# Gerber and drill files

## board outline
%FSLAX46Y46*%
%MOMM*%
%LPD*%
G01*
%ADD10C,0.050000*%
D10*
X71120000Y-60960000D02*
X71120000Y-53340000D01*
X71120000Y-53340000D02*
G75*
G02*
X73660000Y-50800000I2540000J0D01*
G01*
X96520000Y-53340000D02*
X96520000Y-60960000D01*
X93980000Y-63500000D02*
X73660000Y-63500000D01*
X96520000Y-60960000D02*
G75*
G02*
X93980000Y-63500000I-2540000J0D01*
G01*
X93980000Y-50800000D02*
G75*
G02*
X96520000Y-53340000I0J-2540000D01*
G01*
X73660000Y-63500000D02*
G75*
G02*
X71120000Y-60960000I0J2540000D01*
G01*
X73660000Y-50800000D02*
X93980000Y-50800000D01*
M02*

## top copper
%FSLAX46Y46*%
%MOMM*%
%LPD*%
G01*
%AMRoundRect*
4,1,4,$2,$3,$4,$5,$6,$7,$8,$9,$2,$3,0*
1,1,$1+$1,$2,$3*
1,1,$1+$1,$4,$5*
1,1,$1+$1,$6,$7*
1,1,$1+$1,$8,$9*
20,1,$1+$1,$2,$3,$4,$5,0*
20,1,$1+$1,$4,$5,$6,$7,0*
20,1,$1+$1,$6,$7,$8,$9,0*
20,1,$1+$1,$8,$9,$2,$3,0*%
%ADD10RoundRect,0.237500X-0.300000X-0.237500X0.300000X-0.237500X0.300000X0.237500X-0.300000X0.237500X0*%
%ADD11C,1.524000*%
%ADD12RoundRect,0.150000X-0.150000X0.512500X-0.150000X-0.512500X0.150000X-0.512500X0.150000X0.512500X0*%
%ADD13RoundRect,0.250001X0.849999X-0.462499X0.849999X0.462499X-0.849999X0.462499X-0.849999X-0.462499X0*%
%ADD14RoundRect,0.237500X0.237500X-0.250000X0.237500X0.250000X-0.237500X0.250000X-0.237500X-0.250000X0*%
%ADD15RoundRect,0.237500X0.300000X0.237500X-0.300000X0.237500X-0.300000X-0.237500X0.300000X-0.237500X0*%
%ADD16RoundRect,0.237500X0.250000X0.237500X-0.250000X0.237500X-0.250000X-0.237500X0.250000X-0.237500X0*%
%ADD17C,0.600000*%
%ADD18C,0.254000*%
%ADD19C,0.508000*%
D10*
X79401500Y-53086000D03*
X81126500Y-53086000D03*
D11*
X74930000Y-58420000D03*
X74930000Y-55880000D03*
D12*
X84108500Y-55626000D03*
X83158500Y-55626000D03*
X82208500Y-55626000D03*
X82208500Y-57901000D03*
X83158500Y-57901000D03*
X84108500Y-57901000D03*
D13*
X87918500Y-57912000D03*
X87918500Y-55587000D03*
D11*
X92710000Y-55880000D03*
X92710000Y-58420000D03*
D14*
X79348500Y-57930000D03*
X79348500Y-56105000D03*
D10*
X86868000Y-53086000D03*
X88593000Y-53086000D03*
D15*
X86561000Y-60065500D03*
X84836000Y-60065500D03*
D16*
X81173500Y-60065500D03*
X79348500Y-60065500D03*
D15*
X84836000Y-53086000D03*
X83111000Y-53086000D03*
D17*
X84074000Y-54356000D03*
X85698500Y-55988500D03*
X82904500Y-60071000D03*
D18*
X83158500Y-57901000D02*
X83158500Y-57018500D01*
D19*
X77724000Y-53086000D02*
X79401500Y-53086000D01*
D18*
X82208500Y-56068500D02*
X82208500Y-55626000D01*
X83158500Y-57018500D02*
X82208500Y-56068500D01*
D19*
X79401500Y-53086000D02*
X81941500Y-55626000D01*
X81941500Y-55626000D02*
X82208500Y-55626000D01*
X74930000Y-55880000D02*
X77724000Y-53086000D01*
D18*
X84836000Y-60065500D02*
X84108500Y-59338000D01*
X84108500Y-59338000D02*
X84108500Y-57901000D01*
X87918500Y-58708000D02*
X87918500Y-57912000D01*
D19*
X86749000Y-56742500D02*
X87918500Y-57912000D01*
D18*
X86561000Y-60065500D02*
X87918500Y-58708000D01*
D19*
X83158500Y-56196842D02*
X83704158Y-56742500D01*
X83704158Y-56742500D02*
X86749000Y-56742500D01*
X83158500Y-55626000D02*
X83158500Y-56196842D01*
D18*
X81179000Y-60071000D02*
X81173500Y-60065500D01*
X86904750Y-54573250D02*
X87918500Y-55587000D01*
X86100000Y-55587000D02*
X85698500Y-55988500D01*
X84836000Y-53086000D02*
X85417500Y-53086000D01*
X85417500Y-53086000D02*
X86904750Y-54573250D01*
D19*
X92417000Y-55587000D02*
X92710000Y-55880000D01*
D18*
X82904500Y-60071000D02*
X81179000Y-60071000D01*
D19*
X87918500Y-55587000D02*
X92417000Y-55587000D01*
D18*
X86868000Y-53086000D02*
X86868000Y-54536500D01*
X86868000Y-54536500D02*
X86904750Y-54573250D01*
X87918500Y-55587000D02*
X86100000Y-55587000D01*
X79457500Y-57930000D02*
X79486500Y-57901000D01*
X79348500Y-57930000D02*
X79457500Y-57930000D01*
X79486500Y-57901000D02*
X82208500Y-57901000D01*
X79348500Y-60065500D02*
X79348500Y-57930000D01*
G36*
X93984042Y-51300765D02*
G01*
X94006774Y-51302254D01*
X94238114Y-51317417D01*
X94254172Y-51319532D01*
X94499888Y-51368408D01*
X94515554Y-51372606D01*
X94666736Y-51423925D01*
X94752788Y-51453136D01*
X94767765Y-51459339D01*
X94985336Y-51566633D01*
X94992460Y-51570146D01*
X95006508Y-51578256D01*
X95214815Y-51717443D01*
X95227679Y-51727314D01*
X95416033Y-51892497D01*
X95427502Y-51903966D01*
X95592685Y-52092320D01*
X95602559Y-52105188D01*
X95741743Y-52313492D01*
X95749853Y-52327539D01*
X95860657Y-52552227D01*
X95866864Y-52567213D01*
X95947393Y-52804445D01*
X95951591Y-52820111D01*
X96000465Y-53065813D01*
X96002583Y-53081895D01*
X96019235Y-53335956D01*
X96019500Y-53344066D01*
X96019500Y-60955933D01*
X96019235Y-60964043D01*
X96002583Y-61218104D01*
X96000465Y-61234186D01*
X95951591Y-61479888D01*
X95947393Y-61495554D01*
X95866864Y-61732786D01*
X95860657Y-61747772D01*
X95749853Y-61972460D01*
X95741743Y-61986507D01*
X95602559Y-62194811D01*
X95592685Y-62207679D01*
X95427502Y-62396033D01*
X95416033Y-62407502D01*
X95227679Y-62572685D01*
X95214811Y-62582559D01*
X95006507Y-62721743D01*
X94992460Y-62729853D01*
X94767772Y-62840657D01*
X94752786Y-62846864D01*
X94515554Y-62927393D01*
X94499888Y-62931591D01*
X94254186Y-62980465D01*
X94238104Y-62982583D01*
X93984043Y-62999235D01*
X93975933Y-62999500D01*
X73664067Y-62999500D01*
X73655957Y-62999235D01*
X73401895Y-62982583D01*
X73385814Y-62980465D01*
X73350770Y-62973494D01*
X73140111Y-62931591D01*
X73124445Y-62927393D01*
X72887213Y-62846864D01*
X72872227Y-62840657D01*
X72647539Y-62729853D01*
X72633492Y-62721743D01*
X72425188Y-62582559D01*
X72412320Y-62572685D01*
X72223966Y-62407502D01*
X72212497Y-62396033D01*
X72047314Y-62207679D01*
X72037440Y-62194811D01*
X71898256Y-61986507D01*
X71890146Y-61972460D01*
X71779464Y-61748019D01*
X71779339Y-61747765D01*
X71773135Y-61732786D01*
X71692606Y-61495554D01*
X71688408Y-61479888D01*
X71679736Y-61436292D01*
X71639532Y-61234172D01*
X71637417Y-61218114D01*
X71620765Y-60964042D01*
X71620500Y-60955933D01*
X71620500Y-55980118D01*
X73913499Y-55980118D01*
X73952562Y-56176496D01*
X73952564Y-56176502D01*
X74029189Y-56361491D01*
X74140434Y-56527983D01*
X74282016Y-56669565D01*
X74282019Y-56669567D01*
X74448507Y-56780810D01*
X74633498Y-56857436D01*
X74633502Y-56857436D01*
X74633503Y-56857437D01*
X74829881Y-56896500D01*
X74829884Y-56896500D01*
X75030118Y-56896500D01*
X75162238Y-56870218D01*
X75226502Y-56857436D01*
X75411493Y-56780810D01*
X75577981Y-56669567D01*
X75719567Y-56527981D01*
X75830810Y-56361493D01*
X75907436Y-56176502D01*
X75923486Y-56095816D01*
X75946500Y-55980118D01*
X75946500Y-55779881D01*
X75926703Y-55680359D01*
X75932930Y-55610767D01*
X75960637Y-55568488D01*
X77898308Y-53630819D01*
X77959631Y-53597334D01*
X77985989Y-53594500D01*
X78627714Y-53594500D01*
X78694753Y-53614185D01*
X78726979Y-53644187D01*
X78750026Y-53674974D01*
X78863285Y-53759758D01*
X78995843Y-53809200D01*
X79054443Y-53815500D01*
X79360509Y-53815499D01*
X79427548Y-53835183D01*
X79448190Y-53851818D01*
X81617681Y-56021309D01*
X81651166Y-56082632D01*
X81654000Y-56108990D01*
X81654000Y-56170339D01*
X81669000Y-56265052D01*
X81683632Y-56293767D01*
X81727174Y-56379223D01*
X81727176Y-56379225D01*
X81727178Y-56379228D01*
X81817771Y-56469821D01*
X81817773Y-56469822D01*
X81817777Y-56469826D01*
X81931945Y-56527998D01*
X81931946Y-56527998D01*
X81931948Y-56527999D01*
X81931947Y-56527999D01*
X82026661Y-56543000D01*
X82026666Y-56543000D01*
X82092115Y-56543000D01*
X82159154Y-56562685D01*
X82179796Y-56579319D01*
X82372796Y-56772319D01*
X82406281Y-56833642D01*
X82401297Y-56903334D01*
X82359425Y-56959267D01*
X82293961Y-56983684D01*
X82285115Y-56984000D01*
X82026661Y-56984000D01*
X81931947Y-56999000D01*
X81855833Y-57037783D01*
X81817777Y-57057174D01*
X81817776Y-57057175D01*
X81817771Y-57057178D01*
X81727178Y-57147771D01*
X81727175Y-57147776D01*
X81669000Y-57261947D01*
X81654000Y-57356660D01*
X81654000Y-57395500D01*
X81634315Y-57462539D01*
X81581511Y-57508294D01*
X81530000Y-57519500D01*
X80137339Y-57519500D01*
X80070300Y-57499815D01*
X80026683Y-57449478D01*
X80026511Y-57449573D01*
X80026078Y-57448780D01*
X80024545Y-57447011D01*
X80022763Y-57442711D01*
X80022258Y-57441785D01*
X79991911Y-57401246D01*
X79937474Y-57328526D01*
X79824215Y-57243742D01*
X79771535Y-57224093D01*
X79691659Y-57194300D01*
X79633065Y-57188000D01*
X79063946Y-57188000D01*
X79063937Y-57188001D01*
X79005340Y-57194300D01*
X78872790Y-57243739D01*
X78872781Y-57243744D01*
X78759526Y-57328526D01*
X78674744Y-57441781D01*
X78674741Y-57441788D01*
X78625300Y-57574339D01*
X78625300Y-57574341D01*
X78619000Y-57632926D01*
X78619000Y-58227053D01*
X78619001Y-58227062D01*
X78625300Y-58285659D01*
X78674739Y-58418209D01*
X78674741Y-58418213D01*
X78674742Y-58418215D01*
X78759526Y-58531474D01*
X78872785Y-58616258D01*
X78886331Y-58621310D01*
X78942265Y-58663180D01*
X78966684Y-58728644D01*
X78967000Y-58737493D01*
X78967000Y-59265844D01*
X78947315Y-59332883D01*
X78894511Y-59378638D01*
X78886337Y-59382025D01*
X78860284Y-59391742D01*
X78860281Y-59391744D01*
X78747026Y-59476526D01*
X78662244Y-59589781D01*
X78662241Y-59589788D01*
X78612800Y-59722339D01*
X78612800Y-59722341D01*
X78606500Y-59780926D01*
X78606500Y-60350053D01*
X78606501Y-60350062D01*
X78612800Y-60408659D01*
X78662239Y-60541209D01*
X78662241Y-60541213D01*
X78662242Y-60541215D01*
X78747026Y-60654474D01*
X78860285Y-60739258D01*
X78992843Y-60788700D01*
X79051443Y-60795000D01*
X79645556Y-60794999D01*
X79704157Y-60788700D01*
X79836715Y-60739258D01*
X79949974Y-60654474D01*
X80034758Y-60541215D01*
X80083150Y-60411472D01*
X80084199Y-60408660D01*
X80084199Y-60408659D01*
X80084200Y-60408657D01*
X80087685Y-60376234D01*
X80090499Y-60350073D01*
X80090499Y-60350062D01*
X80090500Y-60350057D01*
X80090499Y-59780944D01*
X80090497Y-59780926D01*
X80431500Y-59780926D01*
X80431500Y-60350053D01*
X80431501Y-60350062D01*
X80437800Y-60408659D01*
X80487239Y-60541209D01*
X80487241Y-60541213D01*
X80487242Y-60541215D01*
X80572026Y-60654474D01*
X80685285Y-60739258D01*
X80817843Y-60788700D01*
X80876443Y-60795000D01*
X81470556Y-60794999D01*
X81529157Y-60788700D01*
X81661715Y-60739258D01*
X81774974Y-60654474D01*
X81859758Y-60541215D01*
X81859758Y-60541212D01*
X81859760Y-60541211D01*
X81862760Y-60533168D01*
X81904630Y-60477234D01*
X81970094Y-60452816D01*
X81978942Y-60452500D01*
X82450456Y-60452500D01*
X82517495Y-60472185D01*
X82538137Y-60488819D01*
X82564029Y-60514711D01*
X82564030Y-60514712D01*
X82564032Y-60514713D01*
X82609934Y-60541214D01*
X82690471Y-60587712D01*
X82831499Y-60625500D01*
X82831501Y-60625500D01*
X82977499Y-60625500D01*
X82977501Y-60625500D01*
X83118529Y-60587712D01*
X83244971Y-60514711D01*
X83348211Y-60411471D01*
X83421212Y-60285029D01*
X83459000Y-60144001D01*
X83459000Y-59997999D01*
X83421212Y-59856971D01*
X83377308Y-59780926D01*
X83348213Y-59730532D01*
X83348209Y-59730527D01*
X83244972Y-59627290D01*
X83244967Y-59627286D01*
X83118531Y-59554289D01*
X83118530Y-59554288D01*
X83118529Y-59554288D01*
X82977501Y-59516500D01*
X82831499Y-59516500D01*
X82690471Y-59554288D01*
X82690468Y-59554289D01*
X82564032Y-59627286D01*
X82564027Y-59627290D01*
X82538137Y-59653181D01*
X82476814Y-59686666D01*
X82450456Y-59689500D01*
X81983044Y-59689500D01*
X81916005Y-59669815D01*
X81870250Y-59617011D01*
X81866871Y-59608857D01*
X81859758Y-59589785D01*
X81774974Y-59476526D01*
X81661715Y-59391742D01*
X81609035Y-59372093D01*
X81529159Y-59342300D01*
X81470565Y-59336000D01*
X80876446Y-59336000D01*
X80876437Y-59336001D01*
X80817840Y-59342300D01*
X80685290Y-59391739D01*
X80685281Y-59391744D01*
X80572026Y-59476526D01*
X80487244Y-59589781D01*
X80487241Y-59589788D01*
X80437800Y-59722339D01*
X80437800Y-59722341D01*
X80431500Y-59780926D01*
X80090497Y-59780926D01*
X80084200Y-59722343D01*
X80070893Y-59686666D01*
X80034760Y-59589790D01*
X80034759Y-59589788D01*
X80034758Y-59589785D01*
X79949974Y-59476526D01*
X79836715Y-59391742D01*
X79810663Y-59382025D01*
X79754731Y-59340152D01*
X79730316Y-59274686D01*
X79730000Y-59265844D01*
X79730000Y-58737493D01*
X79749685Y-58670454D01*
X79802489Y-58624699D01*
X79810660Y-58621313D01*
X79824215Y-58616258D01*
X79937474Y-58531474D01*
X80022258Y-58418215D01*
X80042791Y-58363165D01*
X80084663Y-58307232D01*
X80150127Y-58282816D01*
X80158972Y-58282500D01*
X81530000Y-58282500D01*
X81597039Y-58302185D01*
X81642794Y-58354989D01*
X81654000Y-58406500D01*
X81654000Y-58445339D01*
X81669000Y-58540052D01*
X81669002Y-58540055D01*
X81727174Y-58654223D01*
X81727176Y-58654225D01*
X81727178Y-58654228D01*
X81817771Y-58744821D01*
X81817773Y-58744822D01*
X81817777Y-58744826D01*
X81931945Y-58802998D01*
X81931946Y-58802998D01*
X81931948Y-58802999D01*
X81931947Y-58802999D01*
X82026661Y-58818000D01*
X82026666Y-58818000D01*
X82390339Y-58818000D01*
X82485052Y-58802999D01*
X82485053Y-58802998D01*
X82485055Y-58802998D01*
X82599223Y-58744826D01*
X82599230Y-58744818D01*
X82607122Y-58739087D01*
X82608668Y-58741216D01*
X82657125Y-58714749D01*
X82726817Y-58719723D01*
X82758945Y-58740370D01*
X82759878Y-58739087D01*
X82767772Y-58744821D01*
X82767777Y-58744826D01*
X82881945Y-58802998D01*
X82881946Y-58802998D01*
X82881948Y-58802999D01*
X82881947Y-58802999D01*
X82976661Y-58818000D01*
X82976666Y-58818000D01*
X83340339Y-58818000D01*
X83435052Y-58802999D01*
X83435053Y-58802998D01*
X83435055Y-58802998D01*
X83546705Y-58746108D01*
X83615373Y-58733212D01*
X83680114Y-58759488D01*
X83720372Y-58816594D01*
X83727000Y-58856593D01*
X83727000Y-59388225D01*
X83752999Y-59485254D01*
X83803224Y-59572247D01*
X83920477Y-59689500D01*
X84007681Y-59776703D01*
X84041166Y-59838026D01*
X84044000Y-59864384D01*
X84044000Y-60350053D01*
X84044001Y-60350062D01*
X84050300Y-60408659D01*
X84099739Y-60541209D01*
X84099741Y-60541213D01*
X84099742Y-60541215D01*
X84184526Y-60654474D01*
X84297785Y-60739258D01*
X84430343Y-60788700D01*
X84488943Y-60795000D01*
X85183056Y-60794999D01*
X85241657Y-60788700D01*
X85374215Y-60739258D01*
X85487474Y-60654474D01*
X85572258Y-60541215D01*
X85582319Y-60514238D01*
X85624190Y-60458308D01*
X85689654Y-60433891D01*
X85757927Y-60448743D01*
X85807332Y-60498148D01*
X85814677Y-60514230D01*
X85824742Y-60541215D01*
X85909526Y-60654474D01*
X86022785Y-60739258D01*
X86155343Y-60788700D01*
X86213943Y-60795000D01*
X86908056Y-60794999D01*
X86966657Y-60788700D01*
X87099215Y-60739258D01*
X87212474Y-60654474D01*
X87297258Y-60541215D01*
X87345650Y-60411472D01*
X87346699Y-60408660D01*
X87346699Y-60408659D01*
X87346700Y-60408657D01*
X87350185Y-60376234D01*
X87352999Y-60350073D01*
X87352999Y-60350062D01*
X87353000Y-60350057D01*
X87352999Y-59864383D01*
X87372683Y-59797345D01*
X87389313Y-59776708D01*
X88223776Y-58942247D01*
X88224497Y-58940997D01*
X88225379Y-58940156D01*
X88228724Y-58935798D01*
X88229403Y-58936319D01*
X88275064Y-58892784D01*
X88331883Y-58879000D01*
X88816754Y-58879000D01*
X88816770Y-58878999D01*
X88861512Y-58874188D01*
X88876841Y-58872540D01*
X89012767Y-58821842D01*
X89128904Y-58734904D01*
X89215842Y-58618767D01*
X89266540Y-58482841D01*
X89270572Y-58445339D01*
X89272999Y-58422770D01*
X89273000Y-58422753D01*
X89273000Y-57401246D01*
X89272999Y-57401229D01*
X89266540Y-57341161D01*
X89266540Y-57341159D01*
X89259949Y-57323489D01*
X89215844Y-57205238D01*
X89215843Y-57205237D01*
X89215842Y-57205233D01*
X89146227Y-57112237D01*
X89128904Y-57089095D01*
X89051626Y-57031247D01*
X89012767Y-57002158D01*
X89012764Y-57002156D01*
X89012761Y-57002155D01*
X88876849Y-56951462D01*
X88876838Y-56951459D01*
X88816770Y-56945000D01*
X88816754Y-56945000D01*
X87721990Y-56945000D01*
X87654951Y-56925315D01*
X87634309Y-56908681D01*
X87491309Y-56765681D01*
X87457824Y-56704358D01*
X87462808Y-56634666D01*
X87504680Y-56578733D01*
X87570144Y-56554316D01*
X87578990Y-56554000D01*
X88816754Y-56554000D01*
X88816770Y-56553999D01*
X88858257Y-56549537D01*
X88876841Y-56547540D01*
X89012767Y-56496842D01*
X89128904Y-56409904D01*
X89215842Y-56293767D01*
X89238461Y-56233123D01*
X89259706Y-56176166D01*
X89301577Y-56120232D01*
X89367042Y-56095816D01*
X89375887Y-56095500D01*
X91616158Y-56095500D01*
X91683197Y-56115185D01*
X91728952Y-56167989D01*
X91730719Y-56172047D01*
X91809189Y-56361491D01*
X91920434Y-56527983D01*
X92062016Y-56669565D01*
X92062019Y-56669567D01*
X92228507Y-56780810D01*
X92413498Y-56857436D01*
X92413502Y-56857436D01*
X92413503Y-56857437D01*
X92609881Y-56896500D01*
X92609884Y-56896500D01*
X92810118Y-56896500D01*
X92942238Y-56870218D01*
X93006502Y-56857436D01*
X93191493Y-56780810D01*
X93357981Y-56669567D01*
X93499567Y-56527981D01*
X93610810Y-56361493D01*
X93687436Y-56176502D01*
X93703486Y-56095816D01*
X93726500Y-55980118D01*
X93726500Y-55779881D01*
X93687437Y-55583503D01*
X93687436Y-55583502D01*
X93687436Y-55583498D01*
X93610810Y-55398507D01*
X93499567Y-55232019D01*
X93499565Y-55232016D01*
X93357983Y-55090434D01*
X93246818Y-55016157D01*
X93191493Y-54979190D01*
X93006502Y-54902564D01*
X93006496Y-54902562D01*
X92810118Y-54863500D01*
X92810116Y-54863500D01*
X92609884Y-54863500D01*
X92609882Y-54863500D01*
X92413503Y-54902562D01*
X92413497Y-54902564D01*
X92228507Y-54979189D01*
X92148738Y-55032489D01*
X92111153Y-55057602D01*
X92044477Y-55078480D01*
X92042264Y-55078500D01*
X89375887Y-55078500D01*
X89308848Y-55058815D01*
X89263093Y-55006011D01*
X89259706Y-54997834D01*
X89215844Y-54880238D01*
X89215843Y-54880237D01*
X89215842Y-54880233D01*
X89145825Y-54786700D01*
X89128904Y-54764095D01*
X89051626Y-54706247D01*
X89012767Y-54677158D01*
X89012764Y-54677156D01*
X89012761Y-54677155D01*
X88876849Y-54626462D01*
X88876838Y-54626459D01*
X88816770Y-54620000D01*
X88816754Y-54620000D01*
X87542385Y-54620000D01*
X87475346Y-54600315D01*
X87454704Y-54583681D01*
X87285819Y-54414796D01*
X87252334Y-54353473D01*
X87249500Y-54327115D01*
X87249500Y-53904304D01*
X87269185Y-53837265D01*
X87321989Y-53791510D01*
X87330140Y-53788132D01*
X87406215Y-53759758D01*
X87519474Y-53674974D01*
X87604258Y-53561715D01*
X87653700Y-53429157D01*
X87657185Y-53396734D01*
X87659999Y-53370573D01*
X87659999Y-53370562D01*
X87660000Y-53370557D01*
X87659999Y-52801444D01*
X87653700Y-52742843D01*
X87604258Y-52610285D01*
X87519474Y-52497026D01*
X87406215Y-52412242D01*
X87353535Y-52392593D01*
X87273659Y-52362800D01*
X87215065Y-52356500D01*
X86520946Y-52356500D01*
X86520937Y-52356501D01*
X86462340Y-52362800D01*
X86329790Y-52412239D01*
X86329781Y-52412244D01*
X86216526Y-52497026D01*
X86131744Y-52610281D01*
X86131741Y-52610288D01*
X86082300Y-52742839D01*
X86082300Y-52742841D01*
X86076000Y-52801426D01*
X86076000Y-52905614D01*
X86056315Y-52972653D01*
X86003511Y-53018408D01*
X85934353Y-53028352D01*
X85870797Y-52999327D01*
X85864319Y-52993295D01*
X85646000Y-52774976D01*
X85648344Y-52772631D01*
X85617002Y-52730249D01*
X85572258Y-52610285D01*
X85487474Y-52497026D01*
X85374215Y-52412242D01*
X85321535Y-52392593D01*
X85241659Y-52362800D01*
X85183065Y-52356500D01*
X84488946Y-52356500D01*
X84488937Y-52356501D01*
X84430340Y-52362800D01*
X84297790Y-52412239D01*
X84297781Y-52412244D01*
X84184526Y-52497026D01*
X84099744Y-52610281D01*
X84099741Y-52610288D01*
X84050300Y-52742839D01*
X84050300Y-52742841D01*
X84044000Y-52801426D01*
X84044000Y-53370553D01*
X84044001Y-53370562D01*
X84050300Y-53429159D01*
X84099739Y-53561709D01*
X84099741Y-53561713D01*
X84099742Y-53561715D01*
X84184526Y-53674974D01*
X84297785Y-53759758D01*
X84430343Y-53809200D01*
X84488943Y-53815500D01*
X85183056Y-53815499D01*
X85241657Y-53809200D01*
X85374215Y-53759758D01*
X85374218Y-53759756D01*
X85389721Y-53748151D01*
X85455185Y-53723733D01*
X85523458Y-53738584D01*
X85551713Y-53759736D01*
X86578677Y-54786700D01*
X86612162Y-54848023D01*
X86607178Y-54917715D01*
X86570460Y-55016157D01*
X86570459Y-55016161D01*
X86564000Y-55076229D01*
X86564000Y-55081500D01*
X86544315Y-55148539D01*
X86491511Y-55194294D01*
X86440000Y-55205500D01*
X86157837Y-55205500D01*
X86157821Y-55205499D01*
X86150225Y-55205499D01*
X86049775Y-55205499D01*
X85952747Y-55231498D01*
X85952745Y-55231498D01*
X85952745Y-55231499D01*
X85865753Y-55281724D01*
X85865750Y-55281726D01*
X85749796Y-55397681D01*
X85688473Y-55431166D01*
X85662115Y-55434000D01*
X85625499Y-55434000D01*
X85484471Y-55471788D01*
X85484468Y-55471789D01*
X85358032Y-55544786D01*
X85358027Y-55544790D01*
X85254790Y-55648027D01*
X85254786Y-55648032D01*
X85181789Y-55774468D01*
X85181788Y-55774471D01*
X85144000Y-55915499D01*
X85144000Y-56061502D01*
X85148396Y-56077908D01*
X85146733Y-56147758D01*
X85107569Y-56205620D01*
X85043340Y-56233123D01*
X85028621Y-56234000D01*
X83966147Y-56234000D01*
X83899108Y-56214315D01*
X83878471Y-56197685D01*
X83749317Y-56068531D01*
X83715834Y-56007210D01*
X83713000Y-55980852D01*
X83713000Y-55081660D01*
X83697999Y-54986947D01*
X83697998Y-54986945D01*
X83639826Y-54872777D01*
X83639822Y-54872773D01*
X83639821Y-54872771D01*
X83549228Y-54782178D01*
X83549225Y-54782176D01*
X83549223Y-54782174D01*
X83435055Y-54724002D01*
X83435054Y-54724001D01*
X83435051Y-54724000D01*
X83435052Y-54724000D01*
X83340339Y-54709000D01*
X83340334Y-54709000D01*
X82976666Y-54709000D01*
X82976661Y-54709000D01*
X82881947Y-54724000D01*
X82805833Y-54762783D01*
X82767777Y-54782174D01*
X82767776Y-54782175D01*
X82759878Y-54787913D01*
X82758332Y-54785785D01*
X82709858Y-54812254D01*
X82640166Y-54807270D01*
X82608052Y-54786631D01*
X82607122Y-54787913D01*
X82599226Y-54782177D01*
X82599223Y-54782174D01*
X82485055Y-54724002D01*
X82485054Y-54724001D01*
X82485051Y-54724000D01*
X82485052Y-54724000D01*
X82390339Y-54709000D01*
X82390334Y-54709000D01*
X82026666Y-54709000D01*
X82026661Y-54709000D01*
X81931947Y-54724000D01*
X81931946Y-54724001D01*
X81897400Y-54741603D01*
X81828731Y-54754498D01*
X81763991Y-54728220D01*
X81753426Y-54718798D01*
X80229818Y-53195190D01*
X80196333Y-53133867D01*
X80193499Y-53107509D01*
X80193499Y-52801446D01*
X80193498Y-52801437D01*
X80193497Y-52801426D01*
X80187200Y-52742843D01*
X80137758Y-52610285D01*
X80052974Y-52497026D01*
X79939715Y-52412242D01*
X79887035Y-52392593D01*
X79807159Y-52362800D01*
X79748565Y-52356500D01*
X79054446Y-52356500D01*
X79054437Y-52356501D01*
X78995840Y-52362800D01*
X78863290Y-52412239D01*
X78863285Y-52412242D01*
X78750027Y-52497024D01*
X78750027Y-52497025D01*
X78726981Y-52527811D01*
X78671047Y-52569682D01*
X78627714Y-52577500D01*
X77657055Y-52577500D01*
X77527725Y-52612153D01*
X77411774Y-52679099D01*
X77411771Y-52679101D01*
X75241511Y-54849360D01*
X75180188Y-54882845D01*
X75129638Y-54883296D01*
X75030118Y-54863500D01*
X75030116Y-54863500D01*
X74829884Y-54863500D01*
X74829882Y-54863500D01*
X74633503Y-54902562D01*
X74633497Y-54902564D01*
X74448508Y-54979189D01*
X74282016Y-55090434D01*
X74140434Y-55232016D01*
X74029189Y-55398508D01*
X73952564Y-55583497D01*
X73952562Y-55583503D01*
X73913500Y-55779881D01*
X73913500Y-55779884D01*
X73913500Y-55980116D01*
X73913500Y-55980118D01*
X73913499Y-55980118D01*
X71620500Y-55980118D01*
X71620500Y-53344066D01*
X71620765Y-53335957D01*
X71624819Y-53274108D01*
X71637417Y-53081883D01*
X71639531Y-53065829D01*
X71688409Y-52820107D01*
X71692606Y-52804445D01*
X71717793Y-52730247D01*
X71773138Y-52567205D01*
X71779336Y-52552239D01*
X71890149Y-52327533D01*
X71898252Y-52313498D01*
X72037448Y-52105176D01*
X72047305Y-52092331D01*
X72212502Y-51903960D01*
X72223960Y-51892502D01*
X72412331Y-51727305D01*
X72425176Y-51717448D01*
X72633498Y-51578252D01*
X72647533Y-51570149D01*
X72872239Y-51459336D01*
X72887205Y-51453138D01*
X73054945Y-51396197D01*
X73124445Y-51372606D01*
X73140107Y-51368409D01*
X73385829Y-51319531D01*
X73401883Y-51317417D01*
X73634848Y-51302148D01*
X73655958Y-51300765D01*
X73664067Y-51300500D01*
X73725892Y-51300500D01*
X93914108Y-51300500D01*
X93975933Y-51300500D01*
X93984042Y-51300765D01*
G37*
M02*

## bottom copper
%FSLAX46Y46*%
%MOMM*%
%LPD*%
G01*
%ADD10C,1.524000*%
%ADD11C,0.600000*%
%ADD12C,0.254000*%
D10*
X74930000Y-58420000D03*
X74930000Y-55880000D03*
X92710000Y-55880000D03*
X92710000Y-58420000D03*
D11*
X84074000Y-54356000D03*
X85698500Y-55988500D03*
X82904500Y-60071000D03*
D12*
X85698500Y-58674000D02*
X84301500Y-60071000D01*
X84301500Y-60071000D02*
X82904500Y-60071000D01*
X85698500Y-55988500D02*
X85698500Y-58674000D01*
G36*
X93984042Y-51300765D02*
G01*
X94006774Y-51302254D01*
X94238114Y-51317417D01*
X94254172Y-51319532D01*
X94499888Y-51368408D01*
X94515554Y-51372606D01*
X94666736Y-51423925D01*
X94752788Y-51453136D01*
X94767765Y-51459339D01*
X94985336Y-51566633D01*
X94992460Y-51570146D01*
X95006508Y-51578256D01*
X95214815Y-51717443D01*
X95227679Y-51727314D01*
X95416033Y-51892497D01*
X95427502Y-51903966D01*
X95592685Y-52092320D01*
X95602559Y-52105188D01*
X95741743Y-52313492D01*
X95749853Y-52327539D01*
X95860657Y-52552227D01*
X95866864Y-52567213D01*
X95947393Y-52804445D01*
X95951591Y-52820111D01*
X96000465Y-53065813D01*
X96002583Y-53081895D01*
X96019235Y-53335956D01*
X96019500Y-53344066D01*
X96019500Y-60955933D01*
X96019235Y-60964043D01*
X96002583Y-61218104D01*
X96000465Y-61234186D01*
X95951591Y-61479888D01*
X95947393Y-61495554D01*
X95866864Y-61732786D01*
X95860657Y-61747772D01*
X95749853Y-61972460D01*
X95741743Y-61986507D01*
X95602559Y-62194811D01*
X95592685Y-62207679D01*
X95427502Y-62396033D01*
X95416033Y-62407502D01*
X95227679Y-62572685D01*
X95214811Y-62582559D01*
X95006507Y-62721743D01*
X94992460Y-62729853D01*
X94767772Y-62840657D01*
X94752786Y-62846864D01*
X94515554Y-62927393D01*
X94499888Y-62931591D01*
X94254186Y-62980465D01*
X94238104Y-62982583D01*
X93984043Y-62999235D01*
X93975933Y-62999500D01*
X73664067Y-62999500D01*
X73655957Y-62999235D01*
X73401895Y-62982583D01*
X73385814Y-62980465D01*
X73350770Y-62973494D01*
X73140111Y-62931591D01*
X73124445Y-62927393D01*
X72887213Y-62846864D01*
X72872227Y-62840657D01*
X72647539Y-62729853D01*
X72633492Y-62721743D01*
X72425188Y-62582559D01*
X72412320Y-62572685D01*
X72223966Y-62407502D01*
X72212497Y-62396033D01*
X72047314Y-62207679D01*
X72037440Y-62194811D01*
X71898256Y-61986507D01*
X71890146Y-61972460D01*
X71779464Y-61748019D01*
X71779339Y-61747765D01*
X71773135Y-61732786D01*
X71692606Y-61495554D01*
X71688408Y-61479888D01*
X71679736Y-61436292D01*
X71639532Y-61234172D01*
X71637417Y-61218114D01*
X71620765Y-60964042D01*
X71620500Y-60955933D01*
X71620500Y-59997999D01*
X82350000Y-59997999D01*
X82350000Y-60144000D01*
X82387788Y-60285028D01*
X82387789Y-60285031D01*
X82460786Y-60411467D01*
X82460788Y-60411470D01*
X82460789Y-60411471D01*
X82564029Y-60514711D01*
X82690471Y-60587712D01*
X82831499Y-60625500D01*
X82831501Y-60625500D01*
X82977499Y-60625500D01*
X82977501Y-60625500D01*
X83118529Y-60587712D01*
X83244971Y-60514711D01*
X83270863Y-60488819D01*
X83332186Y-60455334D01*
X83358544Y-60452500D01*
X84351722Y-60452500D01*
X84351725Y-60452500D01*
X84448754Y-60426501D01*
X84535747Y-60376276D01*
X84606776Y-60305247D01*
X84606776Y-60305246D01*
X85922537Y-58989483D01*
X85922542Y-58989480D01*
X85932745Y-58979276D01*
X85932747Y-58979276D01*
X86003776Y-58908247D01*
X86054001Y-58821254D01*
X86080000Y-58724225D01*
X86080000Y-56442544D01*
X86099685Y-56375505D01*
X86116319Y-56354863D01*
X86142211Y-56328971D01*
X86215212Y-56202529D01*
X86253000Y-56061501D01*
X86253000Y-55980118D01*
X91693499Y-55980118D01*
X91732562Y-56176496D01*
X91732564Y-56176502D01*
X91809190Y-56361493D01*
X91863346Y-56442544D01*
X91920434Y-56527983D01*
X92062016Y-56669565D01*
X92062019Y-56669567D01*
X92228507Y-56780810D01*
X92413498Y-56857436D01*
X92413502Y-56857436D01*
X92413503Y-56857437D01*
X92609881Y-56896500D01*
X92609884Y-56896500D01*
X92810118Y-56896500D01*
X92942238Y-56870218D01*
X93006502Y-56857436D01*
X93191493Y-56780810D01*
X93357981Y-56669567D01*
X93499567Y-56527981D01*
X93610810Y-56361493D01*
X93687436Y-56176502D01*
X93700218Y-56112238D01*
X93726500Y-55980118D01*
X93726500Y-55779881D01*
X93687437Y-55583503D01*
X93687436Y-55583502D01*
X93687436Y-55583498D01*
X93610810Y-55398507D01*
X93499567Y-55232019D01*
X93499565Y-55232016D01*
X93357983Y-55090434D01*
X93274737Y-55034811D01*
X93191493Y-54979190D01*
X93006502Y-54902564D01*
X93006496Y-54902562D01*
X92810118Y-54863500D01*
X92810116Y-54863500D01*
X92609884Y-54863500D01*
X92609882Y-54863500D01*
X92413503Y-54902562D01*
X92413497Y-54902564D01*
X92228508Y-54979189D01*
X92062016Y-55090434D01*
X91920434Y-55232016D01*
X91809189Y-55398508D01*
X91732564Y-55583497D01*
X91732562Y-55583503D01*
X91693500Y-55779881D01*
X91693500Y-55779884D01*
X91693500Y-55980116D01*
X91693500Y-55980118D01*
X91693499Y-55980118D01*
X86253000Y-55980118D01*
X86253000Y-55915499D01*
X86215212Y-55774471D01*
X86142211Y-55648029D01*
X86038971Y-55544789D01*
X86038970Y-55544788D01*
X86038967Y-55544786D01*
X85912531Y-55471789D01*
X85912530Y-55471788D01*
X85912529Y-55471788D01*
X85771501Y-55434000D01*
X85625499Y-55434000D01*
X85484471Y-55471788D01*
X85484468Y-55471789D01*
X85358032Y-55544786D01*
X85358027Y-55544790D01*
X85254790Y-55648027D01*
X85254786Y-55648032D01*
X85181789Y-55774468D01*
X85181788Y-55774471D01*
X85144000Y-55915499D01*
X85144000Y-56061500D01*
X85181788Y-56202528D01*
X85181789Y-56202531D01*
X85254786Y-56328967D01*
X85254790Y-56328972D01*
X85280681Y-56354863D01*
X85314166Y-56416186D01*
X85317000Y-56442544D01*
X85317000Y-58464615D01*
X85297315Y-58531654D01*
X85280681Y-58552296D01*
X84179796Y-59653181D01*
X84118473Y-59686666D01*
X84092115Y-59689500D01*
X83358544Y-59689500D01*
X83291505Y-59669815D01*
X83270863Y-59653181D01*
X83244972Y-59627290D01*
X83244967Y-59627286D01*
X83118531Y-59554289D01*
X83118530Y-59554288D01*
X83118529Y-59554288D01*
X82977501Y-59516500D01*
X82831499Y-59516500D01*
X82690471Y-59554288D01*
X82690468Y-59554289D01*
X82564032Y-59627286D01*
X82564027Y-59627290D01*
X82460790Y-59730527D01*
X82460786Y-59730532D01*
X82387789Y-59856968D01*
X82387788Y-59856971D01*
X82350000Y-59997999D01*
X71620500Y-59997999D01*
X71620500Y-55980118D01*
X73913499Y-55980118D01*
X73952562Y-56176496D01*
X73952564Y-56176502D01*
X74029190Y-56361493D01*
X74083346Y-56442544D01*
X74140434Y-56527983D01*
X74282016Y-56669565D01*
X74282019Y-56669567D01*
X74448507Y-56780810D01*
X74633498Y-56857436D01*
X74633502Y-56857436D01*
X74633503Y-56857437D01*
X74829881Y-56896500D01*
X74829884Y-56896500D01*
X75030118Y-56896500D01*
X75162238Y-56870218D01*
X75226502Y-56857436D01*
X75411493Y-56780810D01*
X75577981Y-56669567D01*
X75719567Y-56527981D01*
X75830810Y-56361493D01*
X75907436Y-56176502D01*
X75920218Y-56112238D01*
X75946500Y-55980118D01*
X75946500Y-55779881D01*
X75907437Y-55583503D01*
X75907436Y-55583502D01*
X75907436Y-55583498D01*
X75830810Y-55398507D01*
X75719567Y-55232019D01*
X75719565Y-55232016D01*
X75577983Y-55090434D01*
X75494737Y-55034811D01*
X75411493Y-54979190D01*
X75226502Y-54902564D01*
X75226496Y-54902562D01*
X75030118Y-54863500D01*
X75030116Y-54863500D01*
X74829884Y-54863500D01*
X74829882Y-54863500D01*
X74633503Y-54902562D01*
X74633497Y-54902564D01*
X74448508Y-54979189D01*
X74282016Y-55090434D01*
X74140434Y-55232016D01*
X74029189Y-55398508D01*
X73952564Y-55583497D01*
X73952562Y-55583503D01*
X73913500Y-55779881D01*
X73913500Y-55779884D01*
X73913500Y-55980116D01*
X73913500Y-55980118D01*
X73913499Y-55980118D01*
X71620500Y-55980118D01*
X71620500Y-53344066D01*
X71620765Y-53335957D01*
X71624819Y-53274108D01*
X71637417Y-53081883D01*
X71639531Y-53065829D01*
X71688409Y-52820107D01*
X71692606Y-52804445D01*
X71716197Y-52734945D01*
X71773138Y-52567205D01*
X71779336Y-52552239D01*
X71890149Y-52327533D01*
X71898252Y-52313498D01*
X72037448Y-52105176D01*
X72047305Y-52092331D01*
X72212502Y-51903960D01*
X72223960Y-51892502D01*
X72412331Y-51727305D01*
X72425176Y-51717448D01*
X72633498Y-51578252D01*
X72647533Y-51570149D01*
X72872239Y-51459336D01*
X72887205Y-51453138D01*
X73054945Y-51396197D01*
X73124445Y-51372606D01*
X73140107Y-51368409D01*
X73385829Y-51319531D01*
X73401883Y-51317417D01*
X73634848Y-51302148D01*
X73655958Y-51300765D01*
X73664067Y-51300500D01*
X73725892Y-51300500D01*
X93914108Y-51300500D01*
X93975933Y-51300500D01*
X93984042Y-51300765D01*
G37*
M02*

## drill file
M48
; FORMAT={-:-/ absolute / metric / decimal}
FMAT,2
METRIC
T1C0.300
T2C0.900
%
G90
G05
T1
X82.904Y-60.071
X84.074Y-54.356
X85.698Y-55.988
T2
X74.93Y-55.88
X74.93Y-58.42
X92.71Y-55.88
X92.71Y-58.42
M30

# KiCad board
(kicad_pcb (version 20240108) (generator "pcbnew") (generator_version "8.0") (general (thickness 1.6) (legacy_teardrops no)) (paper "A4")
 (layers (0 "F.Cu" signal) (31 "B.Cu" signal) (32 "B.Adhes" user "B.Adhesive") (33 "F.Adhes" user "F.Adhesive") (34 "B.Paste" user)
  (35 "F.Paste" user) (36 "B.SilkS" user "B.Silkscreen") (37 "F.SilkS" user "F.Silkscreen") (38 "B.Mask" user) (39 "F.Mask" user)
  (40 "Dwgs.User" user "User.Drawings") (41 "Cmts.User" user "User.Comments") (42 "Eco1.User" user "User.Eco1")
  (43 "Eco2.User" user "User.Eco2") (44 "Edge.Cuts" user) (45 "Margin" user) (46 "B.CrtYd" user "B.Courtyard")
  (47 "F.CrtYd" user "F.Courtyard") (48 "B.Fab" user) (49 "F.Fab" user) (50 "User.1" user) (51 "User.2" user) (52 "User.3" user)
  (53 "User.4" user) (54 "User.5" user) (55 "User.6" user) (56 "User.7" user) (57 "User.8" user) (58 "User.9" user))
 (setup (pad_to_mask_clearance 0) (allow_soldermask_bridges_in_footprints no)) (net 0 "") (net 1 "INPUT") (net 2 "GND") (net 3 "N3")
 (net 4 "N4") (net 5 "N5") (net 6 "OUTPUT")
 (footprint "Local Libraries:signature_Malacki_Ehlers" (layer "F.Cu") (at 83.312 62.23)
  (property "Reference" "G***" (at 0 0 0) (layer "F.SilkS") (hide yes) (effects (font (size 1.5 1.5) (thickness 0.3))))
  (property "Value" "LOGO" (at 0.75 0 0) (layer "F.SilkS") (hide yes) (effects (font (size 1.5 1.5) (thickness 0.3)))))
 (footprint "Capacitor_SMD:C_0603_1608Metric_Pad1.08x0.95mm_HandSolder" (layer "F.Cu") (at 80.264 53.086)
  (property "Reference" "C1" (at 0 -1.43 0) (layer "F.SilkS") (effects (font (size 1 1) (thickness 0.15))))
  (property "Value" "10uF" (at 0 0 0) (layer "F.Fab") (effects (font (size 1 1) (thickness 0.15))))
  (pad "1" smd roundrect (at -0.8625 0) (size 1.075 0.95) (layers "F.Cu" "F.Paste" "F.Mask") (roundrect_rratio 0.25) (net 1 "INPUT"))
  (pad "2" smd roundrect (at 0.8625 0) (size 1.075 0.95) (layers "F.Cu" "F.Paste" "F.Mask") (roundrect_rratio 0.25) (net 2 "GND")))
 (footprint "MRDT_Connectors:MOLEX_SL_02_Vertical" (layer "F.Cu") (at 74.93 58.42 90)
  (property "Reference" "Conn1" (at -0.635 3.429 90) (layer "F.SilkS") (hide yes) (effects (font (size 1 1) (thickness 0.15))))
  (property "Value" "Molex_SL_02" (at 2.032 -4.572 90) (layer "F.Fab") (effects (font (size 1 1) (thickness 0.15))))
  (pad "1" thru_hole circle (at 0 0 90) (size 1.524 1.524) (drill 0.9) (layers "*.Cu" "*.Mask") (remove_unused_layers no) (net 2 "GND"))
  (pad "2" thru_hole circle (at 2.54 0 90) (size 1.524 1.524) (drill 0.9) (layers "*.Cu" "*.Mask") (remove_unused_layers no) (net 1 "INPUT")))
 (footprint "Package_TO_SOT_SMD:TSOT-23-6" (layer "F.Cu") (at 83.1585 56.7635 -90)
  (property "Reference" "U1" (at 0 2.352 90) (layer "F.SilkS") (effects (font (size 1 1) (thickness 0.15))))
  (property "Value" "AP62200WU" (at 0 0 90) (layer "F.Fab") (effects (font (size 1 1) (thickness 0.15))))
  (pad "1" smd roundrect (at -1.1375 -0.95 270) (size 1.325 0.6) (layers "F.Cu" "F.Paste" "F.Mask") (roundrect_rratio 0.25) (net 2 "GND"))
  (pad "2" smd roundrect (at -1.1375 0 270) (size 1.325 0.6) (layers "F.Cu" "F.Paste" "F.Mask") (roundrect_rratio 0.25) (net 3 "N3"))
  (pad "3" smd roundrect (at -1.1375 0.95 270) (size 1.325 0.6) (layers "F.Cu" "F.Paste" "F.Mask") (roundrect_rratio 0.25) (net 1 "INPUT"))
  (pad "4" smd roundrect (at 1.1375 0.95 270) (size 1.325 0.6) (layers "F.Cu" "F.Paste" "F.Mask") (roundrect_rratio 0.25) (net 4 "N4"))
  (pad "5" smd roundrect (at 1.1375 0 270) (size 1.325 0.6) (layers "F.Cu" "F.Paste" "F.Mask") (roundrect_rratio 0.25) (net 1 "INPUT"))
  (pad "6" smd roundrect (at 1.1375 -0.95 270) (size 1.325 0.6) (layers "F.Cu" "F.Paste" "F.Mask") (roundrect_rratio 0.25) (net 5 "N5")))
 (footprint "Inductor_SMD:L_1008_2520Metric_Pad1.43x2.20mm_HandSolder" (layer "F.Cu") (at 87.9185 56.7495 90)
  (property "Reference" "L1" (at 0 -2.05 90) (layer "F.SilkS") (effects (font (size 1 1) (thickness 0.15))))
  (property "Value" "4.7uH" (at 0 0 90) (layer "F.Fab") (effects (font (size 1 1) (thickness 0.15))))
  (pad "1" smd roundrect (at -1.1625 0 90) (size 1.425 2.2) (layers "F.Cu" "F.Paste" "F.Mask") (roundrect_rratio 0.175439) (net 3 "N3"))
  (pad "2" smd roundrect (at 1.1625 0 90) (size 1.425 2.2) (layers "F.Cu" "F.Paste" "F.Mask") (roundrect_rratio 0.175439) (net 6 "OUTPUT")))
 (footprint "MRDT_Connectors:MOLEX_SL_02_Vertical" (layer "F.Cu") (at 92.71 55.88 -90)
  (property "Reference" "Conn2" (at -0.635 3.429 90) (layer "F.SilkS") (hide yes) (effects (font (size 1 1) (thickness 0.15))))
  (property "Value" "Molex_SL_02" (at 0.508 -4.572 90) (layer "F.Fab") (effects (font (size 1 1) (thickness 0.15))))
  (pad "1" thru_hole circle (at 0 0 270) (size 1.524 1.524) (drill 0.9) (layers "*.Cu" "*.Mask") (remove_unused_layers no) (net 6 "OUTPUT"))
  (pad "2" thru_hole circle (at 2.54 0 270) (size 1.524 1.524) (drill 0.9) (layers "*.Cu" "*.Mask") (remove_unused_layers no) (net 2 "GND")))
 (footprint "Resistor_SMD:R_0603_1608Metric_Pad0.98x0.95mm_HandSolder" (layer "F.Cu") (at 79.3485 57.0175 90)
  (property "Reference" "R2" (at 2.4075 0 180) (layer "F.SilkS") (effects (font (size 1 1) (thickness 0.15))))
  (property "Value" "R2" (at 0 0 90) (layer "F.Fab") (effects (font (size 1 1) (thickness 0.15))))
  (pad "1" smd roundrect (at -0.9125 0 90) (size 0.975 0.95) (layers "F.Cu" "F.Paste" "F.Mask") (roundrect_rratio 0.25) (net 4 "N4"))
  (pad "2" smd roundrect (at 0.9125 0 90) (size 0.975 0.95) (layers "F.Cu" "F.Paste" "F.Mask") (roundrect_rratio 0.25) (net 2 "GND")))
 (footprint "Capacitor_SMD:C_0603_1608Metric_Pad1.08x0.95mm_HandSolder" (layer "F.Cu") (at 87.7305 53.086)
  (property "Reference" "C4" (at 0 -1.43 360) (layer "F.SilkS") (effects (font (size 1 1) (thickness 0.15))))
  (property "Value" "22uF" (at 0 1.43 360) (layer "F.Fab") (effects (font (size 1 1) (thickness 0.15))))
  (pad "1" smd roundrect (at -0.8625 0) (size 1.075 0.95) (layers "F.Cu" "F.Paste" "F.Mask") (roundrect_rratio 0.25) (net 6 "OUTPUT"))
  (pad "2" smd roundrect (at 0.8625 0) (size 1.075 0.95) (layers "F.Cu" "F.Paste" "F.Mask") (roundrect_rratio 0.25) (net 2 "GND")))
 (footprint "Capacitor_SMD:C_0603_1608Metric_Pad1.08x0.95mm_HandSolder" (layer "F.Cu") (at 85.6985 60.0655 180)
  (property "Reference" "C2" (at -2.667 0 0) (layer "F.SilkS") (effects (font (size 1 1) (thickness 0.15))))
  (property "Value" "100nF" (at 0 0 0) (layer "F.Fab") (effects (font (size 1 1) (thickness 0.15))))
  (pad "1" smd roundrect (at -0.8625 0 180) (size 1.075 0.95) (layers "F.Cu" "F.Paste" "F.Mask") (roundrect_rratio 0.25) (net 3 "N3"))
  (pad "2" smd roundrect (at 0.8625 0 180) (size 1.075 0.95) (layers "F.Cu" "F.Paste" "F.Mask") (roundrect_rratio 0.25) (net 5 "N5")))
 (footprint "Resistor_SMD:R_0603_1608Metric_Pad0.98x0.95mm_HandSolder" (layer "F.Cu") (at 80.261 60.0655 180)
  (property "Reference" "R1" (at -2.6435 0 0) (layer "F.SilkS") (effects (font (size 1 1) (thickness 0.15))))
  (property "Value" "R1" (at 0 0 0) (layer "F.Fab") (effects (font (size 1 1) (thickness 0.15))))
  (pad "1" smd roundrect (at -0.9125 0 180) (size 0.975 0.95) (layers "F.Cu" "F.Paste" "F.Mask") (roundrect_rratio 0.25) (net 6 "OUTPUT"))
  (pad "2" smd roundrect (at 0.9125 0 180) (size 0.975 0.95) (layers "F.Cu" "F.Paste" "F.Mask") (roundrect_rratio 0.25) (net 4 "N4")))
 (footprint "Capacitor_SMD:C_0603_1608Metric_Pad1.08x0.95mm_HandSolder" (layer "F.Cu") (at 83.9735 53.086 180)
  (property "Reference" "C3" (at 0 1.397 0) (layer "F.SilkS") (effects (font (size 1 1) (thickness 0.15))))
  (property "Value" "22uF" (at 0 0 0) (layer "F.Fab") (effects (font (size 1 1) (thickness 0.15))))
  (pad "1" smd roundrect (at -0.8625 0 180) (size 1.075 0.95) (layers "F.Cu" "F.Paste" "F.Mask") (roundrect_rratio 0.25) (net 6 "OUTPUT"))
  (pad "2" smd roundrect (at 0.8625 0 180) (size 1.075 0.95) (layers "F.Cu" "F.Paste" "F.Mask") (roundrect_rratio 0.25) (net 2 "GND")))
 (gr_line (start 71.12 60.96) (end 71.12 53.34) (stroke (width 0.05) (type default)) (layer "Edge.Cuts"))
 (gr_arc (start 71.12 53.34) (mid 71.863949 51.543949) (end 73.66 50.8) (stroke (width 0.05) (type default)) (layer "Edge.Cuts"))
 (gr_line (start 96.52 53.34) (end 96.52 60.96) (stroke (width 0.05) (type default)) (layer "Edge.Cuts"))
 (gr_line (start 93.98 63.5) (end 73.66 63.5) (stroke (width 0.05) (type default)) (layer "Edge.Cuts"))
 (gr_arc (start 96.52 60.96) (mid 95.776051 62.756051) (end 93.98 63.5) (stroke (width 0.05) (type default)) (layer "Edge.Cuts"))
 (gr_arc (start 93.98 50.8) (mid 95.776051 51.543949) (end 96.52 53.34) (stroke (width 0.05) (type default)) (layer "Edge.Cuts"))
 (gr_arc (start 73.66 63.5) (mid 71.863949 62.756051) (end 71.12 60.96) (stroke (width 0.05) (type default)) (layer "Edge.Cuts"))
 (gr_line (start 73.66 50.8) (end 93.98 50.8) (stroke (width 0.05) (type default)) (layer "Edge.Cuts"))
 (segment (start 83.1585 57.901) (end 83.1585 57.0185) (width 0.254) (layer "F.Cu") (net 1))
 (segment (start 77.724 53.086) (end 79.4015 53.086) (width 0.508) (layer "F.Cu") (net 1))
 (segment (start 82.2085 56.0685) (end 82.2085 55.626) (width 0.254) (layer "F.Cu") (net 1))
 (segment (start 83.1585 57.0185) (end 82.2085 56.0685) (width 0.254) (layer "F.Cu") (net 1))
 (segment (start 79.4015 53.086) (end 81.9415 55.626) (width 0.508) (layer "F.Cu") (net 1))
 (segment (start 81.9415 55.626) (end 82.2085 55.626) (width 0.508) (layer "F.Cu") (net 1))
 (segment (start 74.93 55.88) (end 77.724 53.086) (width 0.508) (layer "F.Cu") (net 1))
 (via (at 84.074 54.356) (size 0.6) (drill 0.3) (layers "F.Cu" "B.Cu") (free yes) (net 2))
 (segment (start 84.836 60.0655) (end 84.1085 59.338) (width 0.254) (layer "F.Cu") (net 5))
 (segment (start 84.1085 59.338) (end 84.1085 57.901) (width 0.254) (layer "F.Cu") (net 5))
 (segment (start 87.9185 58.708) (end 87.9185 57.912) (width 0.254) (layer "F.Cu") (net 3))
 (segment (start 86.749 56.7425) (end 87.9185 57.912) (width 0.508) (layer "F.Cu") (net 3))
 (segment (start 86.561 60.0655) (end 87.9185 58.708) (width 0.254) (layer "F.Cu") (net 3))
 (segment (start 83.1585 56.196842) (end 83.704158 56.7425) (width 0.508) (layer "F.Cu") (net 3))
 (segment (start 83.704158 56.7425) (end 86.749 56.7425) (width 0.508) (layer "F.Cu") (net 3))
 (segment (start 83.1585 55.626) (end 83.1585 56.196842) (width 0.508) (layer "F.Cu") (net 3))
 (segment (start 81.179 60.071) (end 81.1735 60.0655) (width 0.254) (layer "F.Cu") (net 6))
 (segment (start 86.90475 54.57325) (end 87.9185 55.587) (width 0.254) (layer "F.Cu") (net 6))
 (segment (start 86.1 55.587) (end 85.6985 55.9885) (width 0.254) (layer "F.Cu") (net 6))
 (segment (start 84.836 53.086) (end 85.4175 53.086) (width 0.254) (layer "F.Cu") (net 6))
 (segment (start 85.4175 53.086) (end 86.90475 54.57325) (width 0.254) (layer "F.Cu") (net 6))
 (segment (start 92.417 55.587) (end 92.71 55.88) (width 0.508) (layer "F.Cu") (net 6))
 (segment (start 82.9045 60.071) (end 81.179 60.071) (width 0.254) (layer "F.Cu") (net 6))
 (segment (start 87.9185 55.587) (end 92.417 55.587) (width 0.508) (layer "F.Cu") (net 6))
 (segment (start 86.868 53.086) (end 86.868 54.5365) (width 0.254) (layer "F.Cu") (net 6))
 (segment (start 86.868 54.5365) (end 86.90475 54.57325) (width 0.254) (layer "F.Cu") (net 6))
 (segment (start 87.9185 55.587) (end 86.1 55.587) (width 0.254) (layer "F.Cu") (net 6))
 (via (at 85.6985 55.9885) (size 0.6) (drill 0.3) (layers "F.Cu" "B.Cu") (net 6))
 (via (at 82.9045 60.071) (size 0.6) (drill 0.3) (layers "F.Cu" "B.Cu") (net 6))
 (segment (start 85.6985 58.674) (end 84.3015 60.071) (width 0.254) (layer "B.Cu") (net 6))
 (segment (start 84.3015 60.071) (end 82.9045 60.071) (width 0.254) (layer "B.Cu") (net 6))
 (segment (start 85.6985 55.9885) (end 85.6985 58.674) (width 0.254) (layer "B.Cu") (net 6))
 (segment (start 79.4575 57.93) (end 79.4865 57.901) (width 0.254) (layer "F.Cu") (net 4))
 (segment (start 79.3485 57.93) (end 79.4575 57.93) (width 0.254) (layer "F.Cu") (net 4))
 (segment (start 79.4865 57.901) (end 82.2085 57.901) (width 0.254) (layer "F.Cu") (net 4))
 (segment (start 79.3485 60.0655) (end 79.3485 57.93) (width 0.254) (layer "F.Cu") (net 4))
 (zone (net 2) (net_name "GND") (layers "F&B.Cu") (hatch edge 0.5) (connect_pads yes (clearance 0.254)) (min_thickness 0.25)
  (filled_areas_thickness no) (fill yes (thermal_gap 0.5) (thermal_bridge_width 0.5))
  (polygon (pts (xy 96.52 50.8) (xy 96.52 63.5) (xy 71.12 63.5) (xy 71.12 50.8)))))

